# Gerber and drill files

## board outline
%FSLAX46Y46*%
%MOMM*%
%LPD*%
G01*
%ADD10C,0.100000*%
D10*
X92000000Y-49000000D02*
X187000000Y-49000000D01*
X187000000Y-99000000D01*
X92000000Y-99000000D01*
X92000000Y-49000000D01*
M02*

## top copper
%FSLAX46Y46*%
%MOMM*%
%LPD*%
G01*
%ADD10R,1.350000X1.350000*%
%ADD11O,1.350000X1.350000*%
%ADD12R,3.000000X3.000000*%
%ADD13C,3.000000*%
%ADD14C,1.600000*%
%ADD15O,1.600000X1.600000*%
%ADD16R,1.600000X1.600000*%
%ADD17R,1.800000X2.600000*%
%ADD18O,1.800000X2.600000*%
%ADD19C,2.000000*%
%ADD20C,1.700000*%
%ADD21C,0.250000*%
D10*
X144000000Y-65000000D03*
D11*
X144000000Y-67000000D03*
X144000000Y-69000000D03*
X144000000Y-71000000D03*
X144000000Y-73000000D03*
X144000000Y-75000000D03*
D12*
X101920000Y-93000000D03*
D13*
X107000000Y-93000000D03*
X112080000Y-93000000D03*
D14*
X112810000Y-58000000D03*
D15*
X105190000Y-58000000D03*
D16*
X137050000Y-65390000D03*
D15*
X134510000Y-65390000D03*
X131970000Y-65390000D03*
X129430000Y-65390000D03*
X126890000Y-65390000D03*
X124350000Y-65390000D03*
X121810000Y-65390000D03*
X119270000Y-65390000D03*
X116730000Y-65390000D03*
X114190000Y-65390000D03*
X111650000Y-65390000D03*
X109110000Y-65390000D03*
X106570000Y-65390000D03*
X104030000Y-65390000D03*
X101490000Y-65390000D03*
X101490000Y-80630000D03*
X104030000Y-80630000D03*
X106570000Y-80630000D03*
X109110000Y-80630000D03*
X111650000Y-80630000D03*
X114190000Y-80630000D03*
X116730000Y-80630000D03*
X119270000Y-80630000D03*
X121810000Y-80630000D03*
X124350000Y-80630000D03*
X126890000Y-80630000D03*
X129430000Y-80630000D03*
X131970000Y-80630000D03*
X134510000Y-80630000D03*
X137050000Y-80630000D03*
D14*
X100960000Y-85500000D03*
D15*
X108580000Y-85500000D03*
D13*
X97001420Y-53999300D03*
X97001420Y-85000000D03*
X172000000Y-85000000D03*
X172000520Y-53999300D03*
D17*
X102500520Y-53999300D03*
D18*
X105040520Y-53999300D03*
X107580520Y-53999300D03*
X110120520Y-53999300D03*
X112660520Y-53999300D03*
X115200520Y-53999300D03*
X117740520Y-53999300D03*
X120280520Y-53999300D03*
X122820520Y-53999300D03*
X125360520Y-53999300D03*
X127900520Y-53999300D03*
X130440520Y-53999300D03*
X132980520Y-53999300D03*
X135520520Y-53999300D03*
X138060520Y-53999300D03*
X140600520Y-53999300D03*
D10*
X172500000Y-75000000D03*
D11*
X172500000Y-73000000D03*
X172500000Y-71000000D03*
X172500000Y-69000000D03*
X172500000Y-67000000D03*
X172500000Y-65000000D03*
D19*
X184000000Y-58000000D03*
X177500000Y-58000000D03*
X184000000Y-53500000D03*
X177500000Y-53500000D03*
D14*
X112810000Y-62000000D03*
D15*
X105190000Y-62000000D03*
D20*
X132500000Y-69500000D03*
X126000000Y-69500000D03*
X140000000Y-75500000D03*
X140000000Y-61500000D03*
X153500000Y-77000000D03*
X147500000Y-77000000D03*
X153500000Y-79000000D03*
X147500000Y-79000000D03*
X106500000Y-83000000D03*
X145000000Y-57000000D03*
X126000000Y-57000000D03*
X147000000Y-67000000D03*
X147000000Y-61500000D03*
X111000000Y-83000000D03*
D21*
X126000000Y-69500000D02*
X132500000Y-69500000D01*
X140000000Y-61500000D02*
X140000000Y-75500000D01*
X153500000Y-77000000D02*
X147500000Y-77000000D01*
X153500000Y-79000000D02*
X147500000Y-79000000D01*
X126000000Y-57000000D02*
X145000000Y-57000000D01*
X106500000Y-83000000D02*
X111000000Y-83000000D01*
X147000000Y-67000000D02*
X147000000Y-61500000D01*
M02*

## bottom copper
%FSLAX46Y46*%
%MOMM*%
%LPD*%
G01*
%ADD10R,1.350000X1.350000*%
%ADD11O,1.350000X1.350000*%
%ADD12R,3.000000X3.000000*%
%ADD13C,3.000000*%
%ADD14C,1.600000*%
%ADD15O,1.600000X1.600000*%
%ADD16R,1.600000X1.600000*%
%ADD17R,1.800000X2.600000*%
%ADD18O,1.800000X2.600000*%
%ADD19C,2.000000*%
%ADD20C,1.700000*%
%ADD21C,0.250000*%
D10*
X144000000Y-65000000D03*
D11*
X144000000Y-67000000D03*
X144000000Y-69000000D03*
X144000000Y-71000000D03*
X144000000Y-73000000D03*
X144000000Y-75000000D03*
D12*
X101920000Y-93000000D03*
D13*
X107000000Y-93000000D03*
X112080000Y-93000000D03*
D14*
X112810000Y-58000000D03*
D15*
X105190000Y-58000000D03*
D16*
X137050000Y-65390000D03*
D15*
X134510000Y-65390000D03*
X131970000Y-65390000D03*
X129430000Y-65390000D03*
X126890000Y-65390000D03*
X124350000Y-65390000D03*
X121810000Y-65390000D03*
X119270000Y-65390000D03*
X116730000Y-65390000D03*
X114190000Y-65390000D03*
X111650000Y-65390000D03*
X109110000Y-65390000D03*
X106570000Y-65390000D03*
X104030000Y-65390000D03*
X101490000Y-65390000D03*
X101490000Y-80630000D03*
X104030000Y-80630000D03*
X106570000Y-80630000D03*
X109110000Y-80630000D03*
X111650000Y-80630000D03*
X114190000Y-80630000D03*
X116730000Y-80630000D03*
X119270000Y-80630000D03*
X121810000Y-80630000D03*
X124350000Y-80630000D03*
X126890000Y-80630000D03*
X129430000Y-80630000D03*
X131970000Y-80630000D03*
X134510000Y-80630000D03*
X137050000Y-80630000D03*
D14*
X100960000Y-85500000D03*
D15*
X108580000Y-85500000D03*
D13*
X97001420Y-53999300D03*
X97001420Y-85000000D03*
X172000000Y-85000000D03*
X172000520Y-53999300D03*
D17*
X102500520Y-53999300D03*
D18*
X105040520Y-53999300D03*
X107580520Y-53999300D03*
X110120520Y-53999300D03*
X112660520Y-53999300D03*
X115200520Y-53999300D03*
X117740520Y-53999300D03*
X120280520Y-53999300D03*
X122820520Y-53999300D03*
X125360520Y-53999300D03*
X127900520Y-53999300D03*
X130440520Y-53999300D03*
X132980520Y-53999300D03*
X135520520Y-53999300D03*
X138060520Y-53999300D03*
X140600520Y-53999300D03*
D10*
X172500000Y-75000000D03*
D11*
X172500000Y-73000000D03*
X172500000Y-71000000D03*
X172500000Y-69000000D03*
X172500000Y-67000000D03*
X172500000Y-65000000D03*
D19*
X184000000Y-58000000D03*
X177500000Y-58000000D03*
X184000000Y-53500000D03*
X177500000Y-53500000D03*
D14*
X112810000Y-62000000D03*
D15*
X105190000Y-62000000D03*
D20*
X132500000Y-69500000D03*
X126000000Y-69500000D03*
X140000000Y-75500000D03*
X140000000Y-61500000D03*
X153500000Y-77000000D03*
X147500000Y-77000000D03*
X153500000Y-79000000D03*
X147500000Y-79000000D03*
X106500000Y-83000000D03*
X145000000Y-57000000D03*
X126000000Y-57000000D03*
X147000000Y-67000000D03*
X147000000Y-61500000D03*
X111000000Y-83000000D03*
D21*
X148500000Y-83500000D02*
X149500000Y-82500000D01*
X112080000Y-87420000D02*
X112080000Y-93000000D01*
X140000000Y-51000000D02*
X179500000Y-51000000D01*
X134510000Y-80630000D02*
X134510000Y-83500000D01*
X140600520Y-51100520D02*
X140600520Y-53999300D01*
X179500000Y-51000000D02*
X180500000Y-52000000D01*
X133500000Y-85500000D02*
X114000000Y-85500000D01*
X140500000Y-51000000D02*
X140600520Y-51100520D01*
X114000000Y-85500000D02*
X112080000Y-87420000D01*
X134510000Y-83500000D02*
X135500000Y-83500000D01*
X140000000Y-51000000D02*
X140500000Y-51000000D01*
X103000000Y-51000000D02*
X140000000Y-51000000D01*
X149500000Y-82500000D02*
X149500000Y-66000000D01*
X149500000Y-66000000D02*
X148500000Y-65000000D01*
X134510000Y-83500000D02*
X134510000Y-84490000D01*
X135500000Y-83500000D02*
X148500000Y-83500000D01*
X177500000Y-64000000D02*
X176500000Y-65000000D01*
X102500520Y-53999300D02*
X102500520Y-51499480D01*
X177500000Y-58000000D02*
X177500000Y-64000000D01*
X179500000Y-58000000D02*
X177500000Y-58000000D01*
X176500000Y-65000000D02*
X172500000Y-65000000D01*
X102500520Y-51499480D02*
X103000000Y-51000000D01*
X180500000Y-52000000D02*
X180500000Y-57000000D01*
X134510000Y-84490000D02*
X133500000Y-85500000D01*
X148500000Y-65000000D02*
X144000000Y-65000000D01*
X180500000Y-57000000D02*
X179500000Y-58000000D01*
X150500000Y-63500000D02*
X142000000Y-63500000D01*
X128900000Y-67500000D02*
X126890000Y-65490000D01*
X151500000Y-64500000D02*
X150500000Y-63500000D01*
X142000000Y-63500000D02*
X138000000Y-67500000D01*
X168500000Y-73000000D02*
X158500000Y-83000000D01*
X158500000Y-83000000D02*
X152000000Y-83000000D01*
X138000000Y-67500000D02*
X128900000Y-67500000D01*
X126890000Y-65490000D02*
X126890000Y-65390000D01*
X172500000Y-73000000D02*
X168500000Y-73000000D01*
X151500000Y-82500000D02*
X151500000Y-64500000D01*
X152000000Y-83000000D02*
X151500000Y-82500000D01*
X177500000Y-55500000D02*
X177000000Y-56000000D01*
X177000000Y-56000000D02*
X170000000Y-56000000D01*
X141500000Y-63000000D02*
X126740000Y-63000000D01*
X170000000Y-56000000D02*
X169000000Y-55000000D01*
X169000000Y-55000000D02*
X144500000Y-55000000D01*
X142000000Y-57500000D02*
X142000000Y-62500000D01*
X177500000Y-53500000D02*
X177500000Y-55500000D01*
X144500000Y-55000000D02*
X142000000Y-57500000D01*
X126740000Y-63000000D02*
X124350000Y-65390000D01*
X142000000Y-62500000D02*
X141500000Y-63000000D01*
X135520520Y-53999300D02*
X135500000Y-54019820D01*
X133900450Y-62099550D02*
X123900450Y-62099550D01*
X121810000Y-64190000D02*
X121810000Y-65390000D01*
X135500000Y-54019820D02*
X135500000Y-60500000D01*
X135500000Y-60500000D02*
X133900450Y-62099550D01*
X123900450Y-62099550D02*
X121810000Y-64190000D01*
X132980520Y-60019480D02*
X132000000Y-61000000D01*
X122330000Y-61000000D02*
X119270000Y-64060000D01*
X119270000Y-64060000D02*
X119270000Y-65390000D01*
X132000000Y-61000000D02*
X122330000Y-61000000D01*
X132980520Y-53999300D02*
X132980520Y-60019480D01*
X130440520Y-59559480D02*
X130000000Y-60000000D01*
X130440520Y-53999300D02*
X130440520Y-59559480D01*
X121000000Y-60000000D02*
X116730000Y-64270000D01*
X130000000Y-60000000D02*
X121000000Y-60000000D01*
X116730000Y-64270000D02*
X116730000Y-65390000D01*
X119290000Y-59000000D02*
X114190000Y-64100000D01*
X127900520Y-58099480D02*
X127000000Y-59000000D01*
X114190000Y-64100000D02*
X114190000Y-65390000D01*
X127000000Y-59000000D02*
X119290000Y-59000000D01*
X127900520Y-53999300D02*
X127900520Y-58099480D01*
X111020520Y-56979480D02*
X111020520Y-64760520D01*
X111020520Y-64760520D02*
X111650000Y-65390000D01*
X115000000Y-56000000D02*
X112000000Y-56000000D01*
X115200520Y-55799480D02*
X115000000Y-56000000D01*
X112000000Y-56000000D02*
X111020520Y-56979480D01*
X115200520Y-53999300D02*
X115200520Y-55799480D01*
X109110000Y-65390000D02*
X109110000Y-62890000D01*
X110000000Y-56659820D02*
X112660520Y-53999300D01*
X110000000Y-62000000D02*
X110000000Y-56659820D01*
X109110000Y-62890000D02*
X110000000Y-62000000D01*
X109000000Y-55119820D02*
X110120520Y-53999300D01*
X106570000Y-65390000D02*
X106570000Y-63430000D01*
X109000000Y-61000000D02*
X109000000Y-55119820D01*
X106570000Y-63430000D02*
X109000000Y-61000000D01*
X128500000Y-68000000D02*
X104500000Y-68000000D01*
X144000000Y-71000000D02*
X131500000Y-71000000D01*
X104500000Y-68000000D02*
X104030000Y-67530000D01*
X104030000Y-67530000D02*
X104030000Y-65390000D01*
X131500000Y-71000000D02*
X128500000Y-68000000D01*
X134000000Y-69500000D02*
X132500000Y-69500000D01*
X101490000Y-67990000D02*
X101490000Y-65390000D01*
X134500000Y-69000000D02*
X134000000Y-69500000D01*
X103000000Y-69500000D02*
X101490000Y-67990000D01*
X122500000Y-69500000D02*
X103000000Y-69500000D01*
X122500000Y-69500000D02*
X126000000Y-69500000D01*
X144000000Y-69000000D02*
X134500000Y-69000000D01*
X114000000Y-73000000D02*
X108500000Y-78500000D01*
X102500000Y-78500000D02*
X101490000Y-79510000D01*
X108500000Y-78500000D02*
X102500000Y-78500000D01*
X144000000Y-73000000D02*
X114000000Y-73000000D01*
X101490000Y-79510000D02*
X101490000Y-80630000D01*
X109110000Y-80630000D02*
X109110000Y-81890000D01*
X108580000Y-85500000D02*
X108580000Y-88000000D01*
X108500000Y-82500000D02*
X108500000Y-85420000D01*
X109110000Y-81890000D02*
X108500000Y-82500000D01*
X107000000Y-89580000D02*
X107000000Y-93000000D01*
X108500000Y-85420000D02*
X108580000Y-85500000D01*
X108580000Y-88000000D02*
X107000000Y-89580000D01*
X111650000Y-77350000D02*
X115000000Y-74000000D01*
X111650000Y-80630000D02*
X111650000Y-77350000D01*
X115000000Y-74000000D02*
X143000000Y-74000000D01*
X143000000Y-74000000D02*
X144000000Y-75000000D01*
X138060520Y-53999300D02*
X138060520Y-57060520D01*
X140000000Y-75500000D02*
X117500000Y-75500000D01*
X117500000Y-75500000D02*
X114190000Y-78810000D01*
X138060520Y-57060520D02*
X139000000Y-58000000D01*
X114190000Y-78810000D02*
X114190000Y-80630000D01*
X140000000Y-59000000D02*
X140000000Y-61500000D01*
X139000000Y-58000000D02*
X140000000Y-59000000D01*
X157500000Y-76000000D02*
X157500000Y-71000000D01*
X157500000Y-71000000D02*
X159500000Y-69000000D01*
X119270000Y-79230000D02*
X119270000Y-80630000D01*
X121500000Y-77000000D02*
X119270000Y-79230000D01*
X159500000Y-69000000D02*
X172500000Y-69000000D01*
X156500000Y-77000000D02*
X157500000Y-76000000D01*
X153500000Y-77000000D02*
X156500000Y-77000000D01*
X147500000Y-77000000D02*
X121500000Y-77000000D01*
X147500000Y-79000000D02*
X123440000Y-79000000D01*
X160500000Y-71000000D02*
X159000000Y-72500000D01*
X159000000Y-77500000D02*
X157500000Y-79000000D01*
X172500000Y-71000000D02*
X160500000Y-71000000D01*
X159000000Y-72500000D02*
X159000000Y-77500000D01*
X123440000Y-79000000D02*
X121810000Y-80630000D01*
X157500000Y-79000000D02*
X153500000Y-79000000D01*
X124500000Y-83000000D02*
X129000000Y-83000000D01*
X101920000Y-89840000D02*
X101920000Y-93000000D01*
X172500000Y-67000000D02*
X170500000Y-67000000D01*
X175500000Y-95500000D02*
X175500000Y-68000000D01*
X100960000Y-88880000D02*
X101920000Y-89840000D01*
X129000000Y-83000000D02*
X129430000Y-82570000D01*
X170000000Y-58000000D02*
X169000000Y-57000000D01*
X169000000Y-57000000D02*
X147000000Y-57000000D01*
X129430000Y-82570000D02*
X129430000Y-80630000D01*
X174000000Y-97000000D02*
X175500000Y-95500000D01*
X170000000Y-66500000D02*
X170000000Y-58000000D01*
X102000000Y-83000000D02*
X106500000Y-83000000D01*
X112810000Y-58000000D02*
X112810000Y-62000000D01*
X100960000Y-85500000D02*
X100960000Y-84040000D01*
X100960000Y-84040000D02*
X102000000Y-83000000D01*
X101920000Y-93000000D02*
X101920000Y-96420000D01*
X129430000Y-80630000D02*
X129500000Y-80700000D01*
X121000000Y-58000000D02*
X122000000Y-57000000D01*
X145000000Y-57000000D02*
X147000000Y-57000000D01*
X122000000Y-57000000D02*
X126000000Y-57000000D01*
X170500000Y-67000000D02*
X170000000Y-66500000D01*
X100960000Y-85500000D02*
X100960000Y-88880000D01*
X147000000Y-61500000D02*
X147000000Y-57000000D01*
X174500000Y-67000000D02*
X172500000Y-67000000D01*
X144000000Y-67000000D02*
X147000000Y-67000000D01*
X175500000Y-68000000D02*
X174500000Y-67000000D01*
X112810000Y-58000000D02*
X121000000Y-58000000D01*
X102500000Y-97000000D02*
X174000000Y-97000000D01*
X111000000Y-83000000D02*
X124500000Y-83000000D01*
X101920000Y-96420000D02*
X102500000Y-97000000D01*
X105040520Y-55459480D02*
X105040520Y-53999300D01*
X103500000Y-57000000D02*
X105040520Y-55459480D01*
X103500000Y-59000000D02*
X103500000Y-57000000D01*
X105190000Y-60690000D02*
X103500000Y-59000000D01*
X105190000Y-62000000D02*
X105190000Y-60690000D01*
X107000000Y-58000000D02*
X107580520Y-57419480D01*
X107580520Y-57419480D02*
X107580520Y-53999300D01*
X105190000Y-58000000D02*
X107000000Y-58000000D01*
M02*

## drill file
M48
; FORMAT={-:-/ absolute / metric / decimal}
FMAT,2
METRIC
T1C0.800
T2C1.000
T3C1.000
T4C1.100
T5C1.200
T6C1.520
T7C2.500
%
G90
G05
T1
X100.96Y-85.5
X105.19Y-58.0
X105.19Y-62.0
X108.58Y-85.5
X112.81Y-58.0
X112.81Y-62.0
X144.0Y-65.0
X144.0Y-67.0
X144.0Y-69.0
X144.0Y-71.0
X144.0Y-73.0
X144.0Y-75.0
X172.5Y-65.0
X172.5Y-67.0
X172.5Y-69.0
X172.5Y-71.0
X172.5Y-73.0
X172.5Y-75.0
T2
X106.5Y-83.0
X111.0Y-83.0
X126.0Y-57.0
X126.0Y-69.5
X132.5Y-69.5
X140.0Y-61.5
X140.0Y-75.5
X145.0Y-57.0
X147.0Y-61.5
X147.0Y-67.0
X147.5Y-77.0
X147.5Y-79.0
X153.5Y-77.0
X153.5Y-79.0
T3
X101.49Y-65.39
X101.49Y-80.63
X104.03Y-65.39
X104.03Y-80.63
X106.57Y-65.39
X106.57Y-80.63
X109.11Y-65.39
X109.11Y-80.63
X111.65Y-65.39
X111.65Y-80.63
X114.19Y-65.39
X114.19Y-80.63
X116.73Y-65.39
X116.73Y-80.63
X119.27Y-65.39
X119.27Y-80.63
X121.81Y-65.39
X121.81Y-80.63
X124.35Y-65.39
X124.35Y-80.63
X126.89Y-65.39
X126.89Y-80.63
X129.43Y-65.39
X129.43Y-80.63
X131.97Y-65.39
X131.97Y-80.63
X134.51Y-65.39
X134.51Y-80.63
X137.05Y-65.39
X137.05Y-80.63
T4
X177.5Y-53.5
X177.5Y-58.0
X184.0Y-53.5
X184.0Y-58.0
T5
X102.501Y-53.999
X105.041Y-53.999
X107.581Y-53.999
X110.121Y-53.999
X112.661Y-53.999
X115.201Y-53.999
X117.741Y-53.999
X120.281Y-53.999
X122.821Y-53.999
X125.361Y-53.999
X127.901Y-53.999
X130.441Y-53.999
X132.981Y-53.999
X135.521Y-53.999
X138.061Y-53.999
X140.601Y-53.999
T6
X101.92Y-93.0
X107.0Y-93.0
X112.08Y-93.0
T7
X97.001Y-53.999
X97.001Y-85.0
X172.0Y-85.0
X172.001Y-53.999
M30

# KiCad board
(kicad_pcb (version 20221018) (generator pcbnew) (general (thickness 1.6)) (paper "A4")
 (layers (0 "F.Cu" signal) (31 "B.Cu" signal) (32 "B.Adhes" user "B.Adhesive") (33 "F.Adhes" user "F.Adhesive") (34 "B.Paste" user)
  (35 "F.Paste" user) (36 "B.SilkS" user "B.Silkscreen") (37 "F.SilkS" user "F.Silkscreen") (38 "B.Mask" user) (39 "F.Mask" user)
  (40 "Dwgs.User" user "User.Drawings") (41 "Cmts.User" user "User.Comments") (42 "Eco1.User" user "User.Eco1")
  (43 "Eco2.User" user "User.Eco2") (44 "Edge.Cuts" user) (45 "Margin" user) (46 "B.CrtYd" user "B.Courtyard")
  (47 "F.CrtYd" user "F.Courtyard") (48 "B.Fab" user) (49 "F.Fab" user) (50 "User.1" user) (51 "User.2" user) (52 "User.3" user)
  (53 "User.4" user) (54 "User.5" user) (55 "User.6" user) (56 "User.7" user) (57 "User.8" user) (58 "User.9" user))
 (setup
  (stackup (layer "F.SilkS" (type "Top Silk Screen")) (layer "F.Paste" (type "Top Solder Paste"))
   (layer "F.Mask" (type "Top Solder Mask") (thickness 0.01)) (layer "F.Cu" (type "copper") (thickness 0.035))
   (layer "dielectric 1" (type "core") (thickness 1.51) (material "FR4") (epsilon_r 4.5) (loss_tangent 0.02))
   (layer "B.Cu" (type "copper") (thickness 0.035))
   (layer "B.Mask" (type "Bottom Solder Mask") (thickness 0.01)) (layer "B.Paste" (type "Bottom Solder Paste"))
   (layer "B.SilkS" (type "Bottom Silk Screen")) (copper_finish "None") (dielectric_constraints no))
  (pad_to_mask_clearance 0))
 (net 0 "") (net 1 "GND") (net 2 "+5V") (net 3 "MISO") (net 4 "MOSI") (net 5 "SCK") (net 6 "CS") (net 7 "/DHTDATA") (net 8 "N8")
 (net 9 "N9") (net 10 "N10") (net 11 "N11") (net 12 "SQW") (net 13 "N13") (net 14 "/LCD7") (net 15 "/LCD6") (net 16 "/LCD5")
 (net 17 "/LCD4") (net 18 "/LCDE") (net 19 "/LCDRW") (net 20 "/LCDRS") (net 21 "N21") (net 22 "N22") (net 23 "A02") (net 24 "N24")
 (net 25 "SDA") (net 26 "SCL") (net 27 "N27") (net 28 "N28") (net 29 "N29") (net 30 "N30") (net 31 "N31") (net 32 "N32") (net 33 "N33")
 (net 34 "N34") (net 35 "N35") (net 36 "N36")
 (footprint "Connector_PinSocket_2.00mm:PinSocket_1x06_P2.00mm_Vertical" (layer "F.Cu") (at 144 65)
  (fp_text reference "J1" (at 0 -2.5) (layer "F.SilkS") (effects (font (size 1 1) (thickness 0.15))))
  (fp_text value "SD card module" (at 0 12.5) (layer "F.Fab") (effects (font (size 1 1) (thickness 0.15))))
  (pad "1" thru_hole rect (at 0 0) (size 1.35 1.35) (drill 0.8) (layers "*.Cu" "*.Mask") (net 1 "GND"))
  (pad "2" thru_hole oval (at 0 2) (size 1.35 1.35) (drill 0.8) (layers "*.Cu" "*.Mask") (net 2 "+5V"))
  (pad "3" thru_hole oval (at 0 4) (size 1.35 1.35) (drill 0.8) (layers "*.Cu" "*.Mask") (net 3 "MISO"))
  (pad "4" thru_hole oval (at 0 6) (size 1.35 1.35) (drill 0.8) (layers "*.Cu" "*.Mask") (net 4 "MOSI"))
  (pad "5" thru_hole oval (at 0 8) (size 1.35 1.35) (drill 0.8) (layers "*.Cu" "*.Mask") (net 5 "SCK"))
  (pad "6" thru_hole oval (at 0 10) (size 1.35 1.35) (drill 0.8) (layers "*.Cu" "*.Mask") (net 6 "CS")))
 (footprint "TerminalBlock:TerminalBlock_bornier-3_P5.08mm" (layer "F.Cu") (at 101.92 93)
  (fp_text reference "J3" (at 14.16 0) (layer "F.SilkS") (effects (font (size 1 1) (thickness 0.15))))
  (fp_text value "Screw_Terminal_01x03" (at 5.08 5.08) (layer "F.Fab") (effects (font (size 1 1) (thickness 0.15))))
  (pad "1" thru_hole rect (at 0 0) (size 3 3) (drill 1.52) (layers "*.Cu" "*.Mask") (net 2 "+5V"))
  (pad "2" thru_hole circle (at 5.08 0) (size 3 3) (drill 1.52) (layers "*.Cu" "*.Mask") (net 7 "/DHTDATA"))
  (pad "3" thru_hole circle (at 10.16 0) (size 3 3) (drill 1.52) (layers "*.Cu" "*.Mask") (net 1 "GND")))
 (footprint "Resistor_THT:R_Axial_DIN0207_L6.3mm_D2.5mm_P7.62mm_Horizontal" (layer "F.Cu") (at 112.81 58 180)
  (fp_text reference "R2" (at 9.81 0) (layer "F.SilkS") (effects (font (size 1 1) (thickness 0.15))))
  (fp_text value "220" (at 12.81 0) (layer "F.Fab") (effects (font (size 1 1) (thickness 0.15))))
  (pad "1" thru_hole circle (at 0 0 180) (size 1.6 1.6) (drill 0.8) (layers "*.Cu" "*.Mask") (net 2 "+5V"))
  (pad "2" thru_hole oval (at 7.62 0 180) (size 1.6 1.6) (drill 0.8) (layers "*.Cu" "*.Mask") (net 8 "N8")))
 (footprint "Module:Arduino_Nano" (layer "F.Cu") (at 137.05 65.39 -90)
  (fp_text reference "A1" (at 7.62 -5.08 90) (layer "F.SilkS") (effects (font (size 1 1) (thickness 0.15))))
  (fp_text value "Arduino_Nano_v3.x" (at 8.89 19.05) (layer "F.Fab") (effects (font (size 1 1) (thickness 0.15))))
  (pad "1" thru_hole rect (at 0 0 270) (size 1.6 1.6) (drill 1) (layers "*.Cu" "*.Mask") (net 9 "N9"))
  (pad "2" thru_hole oval (at 0 2.54 270) (size 1.6 1.6) (drill 1) (layers "*.Cu" "*.Mask") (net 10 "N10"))
  (pad "3" thru_hole oval (at 0 5.08 270) (size 1.6 1.6) (drill 1) (layers "*.Cu" "*.Mask") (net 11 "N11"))
  (pad "4" thru_hole oval (at 0 7.62 270) (size 1.6 1.6) (drill 1) (layers "*.Cu" "*.Mask") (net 1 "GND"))
  (pad "5" thru_hole oval (at 0 10.16 270) (size 1.6 1.6) (drill 1) (layers "*.Cu" "*.Mask") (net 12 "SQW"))
  (pad "6" thru_hole oval (at 0 12.7 270) (size 1.6 1.6) (drill 1) (layers "*.Cu" "*.Mask") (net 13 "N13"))
  (pad "7" thru_hole oval (at 0 15.24 270) (size 1.6 1.6) (drill 1) (layers "*.Cu" "*.Mask") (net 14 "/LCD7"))
  (pad "8" thru_hole oval (at 0 17.78 270) (size 1.6 1.6) (drill 1) (layers "*.Cu" "*.Mask") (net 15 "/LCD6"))
  (pad "9" thru_hole oval (at 0 20.32 270) (size 1.6 1.6) (drill 1) (layers "*.Cu" "*.Mask") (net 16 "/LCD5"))
  (pad "10" thru_hole oval (at 0 22.86 270) (size 1.6 1.6) (drill 1) (layers "*.Cu" "*.Mask") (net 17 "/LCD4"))
  (pad "11" thru_hole oval (at 0 25.4 270) (size 1.6 1.6) (drill 1) (layers "*.Cu" "*.Mask") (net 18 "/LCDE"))
  (pad "12" thru_hole oval (at 0 27.94 270) (size 1.6 1.6) (drill 1) (layers "*.Cu" "*.Mask") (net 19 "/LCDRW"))
  (pad "13" thru_hole oval (at 0 30.48 270) (size 1.6 1.6) (drill 1) (layers "*.Cu" "*.Mask") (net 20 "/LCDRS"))
  (pad "14" thru_hole oval (at 0 33.02 270) (size 1.6 1.6) (drill 1) (layers "*.Cu" "*.Mask") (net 4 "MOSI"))
  (pad "15" thru_hole oval (at 0 35.56 270) (size 1.6 1.6) (drill 1) (layers "*.Cu" "*.Mask") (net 3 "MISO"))
  (pad "16" thru_hole oval (at 15.24 35.56 270) (size 1.6 1.6) (drill 1) (layers "*.Cu" "*.Mask") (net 5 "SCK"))
  (pad "17" thru_hole oval (at 15.24 33.02 270) (size 1.6 1.6) (drill 1) (layers "*.Cu" "*.Mask") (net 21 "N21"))
  (pad "18" thru_hole oval (at 15.24 30.48 270) (size 1.6 1.6) (drill 1) (layers "*.Cu" "*.Mask") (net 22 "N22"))
  (pad "19" thru_hole oval (at 15.24 27.94 270) (size 1.6 1.6) (drill 1) (layers "*.Cu" "*.Mask") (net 7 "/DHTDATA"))
  (pad "20" thru_hole oval (at 15.24 25.4 270) (size 1.6 1.6) (drill 1) (layers "*.Cu" "*.Mask") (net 6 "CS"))
  (pad "21" thru_hole oval (at 15.24 22.86 270) (size 1.6 1.6) (drill 1) (layers "*.Cu" "*.Mask") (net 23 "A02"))
  (pad "22" thru_hole oval (at 15.24 20.32 270) (size 1.6 1.6) (drill 1) (layers "*.Cu" "*.Mask") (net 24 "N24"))
  (pad "23" thru_hole oval (at 15.24 17.78 270) (size 1.6 1.6) (drill 1) (layers "*.Cu" "*.Mask") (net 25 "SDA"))
  (pad "24" thru_hole oval (at 15.24 15.24 270) (size 1.6 1.6) (drill 1) (layers "*.Cu" "*.Mask") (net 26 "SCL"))
  (pad "25" thru_hole oval (at 15.24 12.7 270) (size 1.6 1.6) (drill 1) (layers "*.Cu" "*.Mask") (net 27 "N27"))
  (pad "26" thru_hole oval (at 15.24 10.16 270) (size 1.6 1.6) (drill 1) (layers "*.Cu" "*.Mask") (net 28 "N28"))
  (pad "27" thru_hole oval (at 15.24 7.62 270) (size 1.6 1.6) (drill 1) (layers "*.Cu" "*.Mask") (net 2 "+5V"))
  (pad "28" thru_hole oval (at 15.24 5.08 270) (size 1.6 1.6) (drill 1) (layers "*.Cu" "*.Mask") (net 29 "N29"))
  (pad "29" thru_hole oval (at 15.24 2.54 270) (size 1.6 1.6) (drill 1) (layers "*.Cu" "*.Mask") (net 1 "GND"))
  (pad "30" thru_hole oval (at 15.24 0 270) (size 1.6 1.6) (drill 1) (layers "*.Cu" "*.Mask") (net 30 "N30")))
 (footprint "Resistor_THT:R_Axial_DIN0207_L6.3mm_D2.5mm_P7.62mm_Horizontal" (layer "F.Cu") (at 100.96 85.5)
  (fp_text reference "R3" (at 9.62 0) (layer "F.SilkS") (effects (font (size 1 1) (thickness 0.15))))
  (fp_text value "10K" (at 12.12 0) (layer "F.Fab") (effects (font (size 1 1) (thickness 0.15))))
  (pad "1" thru_hole circle (at 0 0) (size 1.6 1.6) (drill 0.8) (layers "*.Cu" "*.Mask") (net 2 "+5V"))
  (pad "2" thru_hole oval (at 7.62 0) (size 1.6 1.6) (drill 0.8) (layers "*.Cu" "*.Mask") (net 7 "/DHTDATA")))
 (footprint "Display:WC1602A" (layer "F.Cu") (at 102.50052 53.9993)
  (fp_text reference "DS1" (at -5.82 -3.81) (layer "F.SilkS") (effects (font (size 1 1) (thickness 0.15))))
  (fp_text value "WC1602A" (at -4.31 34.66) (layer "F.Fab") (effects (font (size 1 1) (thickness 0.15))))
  (pad "" thru_hole circle (at -5.4991 0) (size 3 3) (drill 2.5) (layers "*.Cu" "*.Mask"))
  (pad "" thru_hole circle (at -5.4991 31.0007) (size 3 3) (drill 2.5) (layers "*.Cu" "*.Mask"))
  (pad "" thru_hole circle (at 69.49948 31.0007) (size 3 3) (drill 2.5) (layers "*.Cu" "*.Mask"))
  (pad "" thru_hole circle (at 69.5 0) (size 3 3) (drill 2.5) (layers "*.Cu" "*.Mask"))
  (pad "1" thru_hole rect (at 0 0) (size 1.8 2.6) (drill 1.2) (layers "*.Cu" "*.Mask") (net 1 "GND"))
  (pad "2" thru_hole oval (at 2.54 0) (size 1.8 2.6) (drill 1.2) (layers "*.Cu" "*.Mask") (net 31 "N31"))
  (pad "3" thru_hole oval (at 5.08 0) (size 1.8 2.6) (drill 1.2) (layers "*.Cu" "*.Mask") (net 8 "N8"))
  (pad "4" thru_hole oval (at 7.62 0) (size 1.8 2.6) (drill 1.2) (layers "*.Cu" "*.Mask") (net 20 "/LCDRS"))
  (pad "5" thru_hole oval (at 10.16 0) (size 1.8 2.6) (drill 1.2) (layers "*.Cu" "*.Mask") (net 19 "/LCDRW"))
  (pad "6" thru_hole oval (at 12.7 0) (size 1.8 2.6) (drill 1.2) (layers "*.Cu" "*.Mask") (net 18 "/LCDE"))
  (pad "7" thru_hole oval (at 15.24 0) (size 1.8 2.6) (drill 1.2) (layers "*.Cu" "*.Mask") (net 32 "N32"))
  (pad "8" thru_hole oval (at 17.78 0) (size 1.8 2.6) (drill 1.2) (layers "*.Cu" "*.Mask") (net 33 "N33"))
  (pad "9" thru_hole oval (at 20.32 0) (size 1.8 2.6) (drill 1.2) (layers "*.Cu" "*.Mask") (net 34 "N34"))
  (pad "10" thru_hole oval (at 22.86 0) (size 1.8 2.6) (drill 1.2) (layers "*.Cu" "*.Mask") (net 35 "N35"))
  (pad "11" thru_hole oval (at 25.4 0) (size 1.8 2.6) (drill 1.2) (layers "*.Cu" "*.Mask") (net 17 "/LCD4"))
  (pad "12" thru_hole oval (at 27.94 0) (size 1.8 2.6) (drill 1.2) (layers "*.Cu" "*.Mask") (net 16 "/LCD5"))
  (pad "13" thru_hole oval (at 30.48 0) (size 1.8 2.6) (drill 1.2) (layers "*.Cu" "*.Mask") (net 15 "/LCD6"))
  (pad "14" thru_hole oval (at 33.02 0) (size 1.8 2.6) (drill 1.2) (layers "*.Cu" "*.Mask") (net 14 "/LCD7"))
  (pad "15" thru_hole oval (at 35.56 0) (size 1.8 2.6) (drill 1.2) (layers "*.Cu" "*.Mask") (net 23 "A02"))
  (pad "16" thru_hole oval (at 38.1 0) (size 1.8 2.6) (drill 1.2) (layers "*.Cu" "*.Mask") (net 1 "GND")))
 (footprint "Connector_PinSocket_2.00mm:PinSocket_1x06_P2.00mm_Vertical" (layer "F.Cu") (at 172.5 75 180)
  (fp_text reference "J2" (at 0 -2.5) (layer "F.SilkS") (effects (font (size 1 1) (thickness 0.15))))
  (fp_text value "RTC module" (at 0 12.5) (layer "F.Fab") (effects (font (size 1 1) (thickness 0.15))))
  (pad "1" thru_hole rect (at 0 0 180) (size 1.35 1.35) (drill 0.8) (layers "*.Cu" "*.Mask") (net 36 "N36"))
  (pad "2" thru_hole oval (at 0 2 180) (size 1.35 1.35) (drill 0.8) (layers "*.Cu" "*.Mask") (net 12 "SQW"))
  (pad "3" thru_hole oval (at 0 4 180) (size 1.35 1.35) (drill 0.8) (layers "*.Cu" "*.Mask") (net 26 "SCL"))
  (pad "4" thru_hole oval (at 0 6 180) (size 1.35 1.35) (drill 0.8) (layers "*.Cu" "*.Mask") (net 25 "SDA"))
  (pad "5" thru_hole oval (at 0 8 180) (size 1.35 1.35) (drill 0.8) (layers "*.Cu" "*.Mask") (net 2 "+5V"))
  (pad "6" thru_hole oval (at 0 10 180) (size 1.35 1.35) (drill 0.8) (layers "*.Cu" "*.Mask") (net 1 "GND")))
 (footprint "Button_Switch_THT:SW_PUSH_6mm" (layer "F.Cu") (at 184 58 180)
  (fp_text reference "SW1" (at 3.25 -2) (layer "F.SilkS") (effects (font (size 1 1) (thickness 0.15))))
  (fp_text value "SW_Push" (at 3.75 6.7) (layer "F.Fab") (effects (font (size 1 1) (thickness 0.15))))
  (pad "1" thru_hole circle (at 0 0 270) (size 2 2) (drill 1.1) (layers "*.Cu" "*.Mask") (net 1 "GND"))
  (pad "1" thru_hole circle (at 6.5 0 270) (size 2 2) (drill 1.1) (layers "*.Cu" "*.Mask") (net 1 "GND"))
  (pad "2" thru_hole circle (at 0 4.5 270) (size 2 2) (drill 1.1) (layers "*.Cu" "*.Mask") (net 13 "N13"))
  (pad "2" thru_hole circle (at 6.5 4.5 270) (size 2 2) (drill 1.1) (layers "*.Cu" "*.Mask") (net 13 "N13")))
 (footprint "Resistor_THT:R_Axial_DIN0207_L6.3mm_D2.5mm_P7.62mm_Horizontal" (layer "F.Cu") (at 112.81 62 180)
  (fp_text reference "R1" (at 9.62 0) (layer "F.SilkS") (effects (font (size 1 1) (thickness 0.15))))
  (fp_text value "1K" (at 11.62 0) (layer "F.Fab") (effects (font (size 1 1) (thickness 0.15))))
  (pad "1" thru_hole circle (at 0 0 180) (size 1.6 1.6) (drill 0.8) (layers "*.Cu" "*.Mask") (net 2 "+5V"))
  (pad "2" thru_hole oval (at 7.62 0 180) (size 1.6 1.6) (drill 0.8) (layers "*.Cu" "*.Mask") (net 31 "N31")))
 (gr_rect (start 92 49) (end 187 99) (stroke (width 0.1) (type default)) (fill none) (layer "Edge.Cuts"))
 (segment (start 148.5 83.5) (end 149.5 82.5) (width 0.25) (layer "B.Cu") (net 1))
 (segment (start 112.08 87.42) (end 112.08 93) (width 0.25) (layer "B.Cu") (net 1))
 (segment (start 140 51) (end 179.5 51) (width 0.25) (layer "B.Cu") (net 1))
 (segment (start 134.51 80.63) (end 134.51 83.5) (width 0.25) (layer "B.Cu") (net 1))
 (segment (start 140.60052 51.10052) (end 140.60052 53.9993) (width 0.25) (layer "B.Cu") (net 1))
 (segment (start 179.5 51) (end 180.5 52) (width 0.25) (layer "B.Cu") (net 1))
 (segment (start 133.5 85.5) (end 114 85.5) (width 0.25) (layer "B.Cu") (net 1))
 (segment (start 140.5 51) (end 140.60052 51.10052) (width 0.25) (layer "B.Cu") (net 1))
 (segment (start 114 85.5) (end 112.08 87.42) (width 0.25) (layer "B.Cu") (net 1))
 (segment (start 134.51 83.5) (end 135.5 83.5) (width 0.25) (layer "B.Cu") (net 1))
 (segment (start 140 51) (end 140.5 51) (width 0.25) (layer "B.Cu") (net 1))
 (segment (start 103 51) (end 140 51) (width 0.25) (layer "B.Cu") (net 1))
 (segment (start 149.5 82.5) (end 149.5 66) (width 0.25) (layer "B.Cu") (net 1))
 (segment (start 149.5 66) (end 148.5 65) (width 0.25) (layer "B.Cu") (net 1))
 (segment (start 134.51 83.5) (end 134.51 84.49) (width 0.25) (layer "B.Cu") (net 1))
 (segment (start 135.5 83.5) (end 148.5 83.5) (width 0.25) (layer "B.Cu") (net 1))
 (segment (start 177.5 64) (end 176.5 65) (width 0.25) (layer "B.Cu") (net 1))
 (segment (start 102.50052 53.9993) (end 102.50052 51.49948) (width 0.25) (layer "B.Cu") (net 1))
 (segment (start 177.5 58) (end 177.5 64) (width 0.25) (layer "B.Cu") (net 1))
 (segment (start 179.5 58) (end 177.5 58) (width 0.25) (layer "B.Cu") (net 1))
 (segment (start 176.5 65) (end 172.5 65) (width 0.25) (layer "B.Cu") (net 1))
 (segment (start 102.50052 51.49948) (end 103 51) (width 0.25) (layer "B.Cu") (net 1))
 (segment (start 180.5 52) (end 180.5 57) (width 0.25) (layer "B.Cu") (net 1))
 (segment (start 134.51 84.49) (end 133.5 85.5) (width 0.25) (layer "B.Cu") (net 1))
 (segment (start 148.5 65) (end 144 65) (width 0.25) (layer "B.Cu") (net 1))
 (segment (start 180.5 57) (end 179.5 58) (width 0.25) (layer "B.Cu") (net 1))
 (segment (start 150.5 63.5) (end 142 63.5) (width 0.25) (layer "B.Cu") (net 12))
 (segment (start 128.9 67.5) (end 126.89 65.49) (width 0.25) (layer "B.Cu") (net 12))
 (segment (start 151.5 64.5) (end 150.5 63.5) (width 0.25) (layer "B.Cu") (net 12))
 (segment (start 142 63.5) (end 138 67.5) (width 0.25) (layer "B.Cu") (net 12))
 (segment (start 168.5 73) (end 158.5 83) (width 0.25) (layer "B.Cu") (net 12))
 (segment (start 158.5 83) (end 152 83) (width 0.25) (layer "B.Cu") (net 12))
 (segment (start 138 67.5) (end 128.9 67.5) (width 0.25) (layer "B.Cu") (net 12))
 (segment (start 126.89 65.49) (end 126.89 65.39) (width 0.25) (layer "B.Cu") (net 12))
 (segment (start 172.5 73) (end 168.5 73) (width 0.25) (layer "B.Cu") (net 12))
 (segment (start 151.5 82.5) (end 151.5 64.5) (width 0.25) (layer "B.Cu") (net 12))
 (segment (start 152 83) (end 151.5 82.5) (width 0.25) (layer "B.Cu") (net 12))
 (segment (start 177.5 55.5) (end 177 56) (width 0.25) (layer "B.Cu") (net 13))
 (segment (start 177 56) (end 170 56) (width 0.25) (layer "B.Cu") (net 13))
 (segment (start 141.5 63) (end 126.74 63) (width 0.25) (layer "B.Cu") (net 13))
 (segment (start 170 56) (end 169 55) (width 0.25) (layer "B.Cu") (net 13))
 (segment (start 169 55) (end 144.5 55) (width 0.25) (layer "B.Cu") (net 13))
 (segment (start 142 57.5) (end 142 62.5) (width 0.25) (layer "B.Cu") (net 13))
 (segment (start 177.5 53.5) (end 177.5 55.5) (width 0.25) (layer "B.Cu") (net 13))
 (segment (start 144.5 55) (end 142 57.5) (width 0.25) (layer "B.Cu") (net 13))
 (segment (start 126.74 63) (end 124.35 65.39) (width 0.25) (layer "B.Cu") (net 13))
 (segment (start 142 62.5) (end 141.5 63) (width 0.25) (layer "B.Cu") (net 13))
 (segment (start 135.52052 53.9993) (end 135.5 54.01982) (width 0.25) (layer "B.Cu") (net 14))
 (segment (start 133.90045 62.09955) (end 123.90045 62.09955) (width 0.25) (layer "B.Cu") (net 14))
 (segment (start 121.81 64.19) (end 121.81 65.39) (width 0.25) (layer "B.Cu") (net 14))
 (segment (start 135.5 54.01982) (end 135.5 60.5) (width 0.25) (layer "B.Cu") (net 14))
 (segment (start 135.5 60.5) (end 133.90045 62.09955) (width 0.25) (layer "B.Cu") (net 14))
 (segment (start 123.90045 62.09955) (end 121.81 64.19) (width 0.25) (layer "B.Cu") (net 14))
 (segment (start 132.98052 60.01948) (end 132 61) (width 0.25) (layer "B.Cu") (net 15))
 (segment (start 122.33 61) (end 119.27 64.06) (width 0.25) (layer "B.Cu") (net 15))
 (segment (start 119.27 64.06) (end 119.27 65.39) (width 0.25) (layer "B.Cu") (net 15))
 (segment (start 132 61) (end 122.33 61) (width 0.25) (layer "B.Cu") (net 15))
 (segment (start 132.98052 53.9993) (end 132.98052 60.01948) (width 0.25) (layer "B.Cu") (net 15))
 (segment (start 130.44052 59.55948) (end 130 60) (width 0.25) (layer "B.Cu") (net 16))
 (segment (start 130.44052 53.9993) (end 130.44052 59.55948) (width 0.25) (layer "B.Cu") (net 16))
 (segment (start 121 60) (end 116.73 64.27) (width 0.25) (layer "B.Cu") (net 16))
 (segment (start 130 60) (end 121 60) (width 0.25) (layer "B.Cu") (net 16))
 (segment (start 116.73 64.27) (end 116.73 65.39) (width 0.25) (layer "B.Cu") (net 16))
 (segment (start 119.29 59) (end 114.19 64.1) (width 0.25) (layer "B.Cu") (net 17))
 (segment (start 127.90052 58.09948) (end 127 59) (width 0.25) (layer "B.Cu") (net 17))
 (segment (start 114.19 64.1) (end 114.19 65.39) (width 0.25) (layer "B.Cu") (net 17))
 (segment (start 127 59) (end 119.29 59) (width 0.25) (layer "B.Cu") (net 17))
 (segment (start 127.90052 53.9993) (end 127.90052 58.09948) (width 0.25) (layer "B.Cu") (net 17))
 (segment (start 111.02052 56.97948) (end 111.02052 64.76052) (width 0.25) (layer "B.Cu") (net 18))
 (segment (start 111.02052 64.76052) (end 111.65 65.39) (width 0.25) (layer "B.Cu") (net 18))
 (segment (start 115 56) (end 112 56) (width 0.25) (layer "B.Cu") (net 18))
 (segment (start 115.20052 55.79948) (end 115 56) (width 0.25) (layer "B.Cu") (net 18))
 (segment (start 112 56) (end 111.02052 56.97948) (width 0.25) (layer "B.Cu") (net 18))
 (segment (start 115.20052 53.9993) (end 115.20052 55.79948) (width 0.25) (layer "B.Cu") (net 18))
 (segment (start 109.11 65.39) (end 109.11 62.89) (width 0.25) (layer "B.Cu") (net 19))
 (segment (start 110 56.65982) (end 112.66052 53.9993) (width 0.25) (layer "B.Cu") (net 19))
 (segment (start 110 62) (end 110 56.65982) (width 0.25) (layer "B.Cu") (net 19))
 (segment (start 109.11 62.89) (end 110 62) (width 0.25) (layer "B.Cu") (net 19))
 (segment (start 109 55.11982) (end 110.12052 53.9993) (width 0.25) (layer "B.Cu") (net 20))
 (segment (start 106.57 65.39) (end 106.57 63.43) (width 0.25) (layer "B.Cu") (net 20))
 (segment (start 109 61) (end 109 55.11982) (width 0.25) (layer "B.Cu") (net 20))
 (segment (start 106.57 63.43) (end 109 61) (width 0.25) (layer "B.Cu") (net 20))
 (segment (start 128.5 68) (end 104.5 68) (width 0.25) (layer "B.Cu") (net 4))
 (segment (start 144 71) (end 131.5 71) (width 0.25) (layer "B.Cu") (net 4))
 (segment (start 104.5 68) (end 104.03 67.53) (width 0.25) (layer "B.Cu") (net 4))
 (segment (start 104.03 67.53) (end 104.03 65.39) (width 0.25) (layer "B.Cu") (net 4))
 (segment (start 131.5 71) (end 128.5 68) (width 0.25) (layer "B.Cu") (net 4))
 (segment (start 126 69.5) (end 132.5 69.5) (width 0.25) (layer "F.Cu") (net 3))
 (via (at 132.5 69.5) (size 1.7) (drill 1) (layers "F.Cu" "B.Cu") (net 3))
 (via (at 126 69.5) (size 1.7) (drill 1) (layers "F.Cu" "B.Cu") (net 3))
 (segment (start 134 69.5) (end 132.5 69.5) (width 0.25) (layer "B.Cu") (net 3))
 (segment (start 101.49 67.99) (end 101.49 65.39) (width 0.25) (layer "B.Cu") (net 3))
 (segment (start 134.5 69) (end 134 69.5) (width 0.25) (layer "B.Cu") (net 3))
 (segment (start 103 69.5) (end 101.49 67.99) (width 0.25) (layer "B.Cu") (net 3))
 (segment (start 122.5 69.5) (end 103 69.5) (width 0.25) (layer "B.Cu") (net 3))
 (segment (start 122.5 69.5) (end 126 69.5) (width 0.25) (layer "B.Cu") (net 3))
 (segment (start 144 69) (end 134.5 69) (width 0.25) (layer "B.Cu") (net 3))
 (segment (start 114 73) (end 108.5 78.5) (width 0.25) (layer "B.Cu") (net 5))
 (segment (start 102.5 78.5) (end 101.49 79.51) (width 0.25) (layer "B.Cu") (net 5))
 (segment (start 108.5 78.5) (end 102.5 78.5) (width 0.25) (layer "B.Cu") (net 5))
 (segment (start 144 73) (end 114 73) (width 0.25) (layer "B.Cu") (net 5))
 (segment (start 101.49 79.51) (end 101.49 80.63) (width 0.25) (layer "B.Cu") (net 5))
 (segment (start 109.11 80.63) (end 109.11 81.89) (width 0.25) (layer "B.Cu") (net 7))
 (segment (start 108.58 85.5) (end 108.58 88) (width 0.25) (layer "B.Cu") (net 7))
 (segment (start 108.5 82.5) (end 108.5 85.42) (width 0.25) (layer "B.Cu") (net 7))
 (segment (start 109.11 81.89) (end 108.5 82.5) (width 0.25) (layer "B.Cu") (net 7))
 (segment (start 107 89.58) (end 107 93) (width 0.25) (layer "B.Cu") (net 7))
 (segment (start 108.5 85.42) (end 108.58 85.5) (width 0.25) (layer "B.Cu") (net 7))
 (segment (start 108.58 88) (end 107 89.58) (width 0.25) (layer "B.Cu") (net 7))
 (segment (start 111.65 77.35) (end 115 74) (width 0.25) (layer "B.Cu") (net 6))
 (segment (start 111.65 80.63) (end 111.65 77.35) (width 0.25) (layer "B.Cu") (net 6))
 (segment (start 115 74) (end 143 74) (width 0.25) (layer "B.Cu") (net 6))
 (segment (start 143 74) (end 144 75) (width 0.25) (layer "B.Cu") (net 6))
 (segment (start 140 61.5) (end 140 75.5) (width 0.25) (layer "F.Cu") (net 23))
 (via (at 140 75.5) (size 1.7) (drill 1) (layers "F.Cu" "B.Cu") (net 23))
 (via (at 140 61.5) (size 1.7) (drill 1) (layers "F.Cu" "B.Cu") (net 23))
 (segment (start 138.06052 53.9993) (end 138.06052 57.06052) (width 0.25) (layer "B.Cu") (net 23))
 (segment (start 140 75.5) (end 117.5 75.5) (width 0.25) (layer "B.Cu") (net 23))
 (segment (start 117.5 75.5) (end 114.19 78.81) (width 0.25) (layer "B.Cu") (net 23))
 (segment (start 138.06052 57.06052) (end 139 58) (width 0.25) (layer "B.Cu") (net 23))
 (segment (start 114.19 78.81) (end 114.19 80.63) (width 0.25) (layer "B.Cu") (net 23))
 (segment (start 140 59) (end 140 61.5) (width 0.25) (layer "B.Cu") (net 23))
 (segment (start 139 58) (end 140 59) (width 0.25) (layer "B.Cu") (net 23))
 (segment (start 153.5 77) (end 147.5 77) (width 0.25) (layer "F.Cu") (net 25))
 (via (at 153.5 77) (size 1.7) (drill 1) (layers "F.Cu" "B.Cu") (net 25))
 (via (at 147.5 77) (size 1.7) (drill 1) (layers "F.Cu" "B.Cu") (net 25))
 (segment (start 157.5 76) (end 157.5 71) (width 0.25) (layer "B.Cu") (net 25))
 (segment (start 157.5 71) (end 159.5 69) (width 0.25) (layer "B.Cu") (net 25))
 (segment (start 119.27 79.23) (end 119.27 80.63) (width 0.25) (layer "B.Cu") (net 25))
 (segment (start 121.5 77) (end 119.27 79.23) (width 0.25) (layer "B.Cu") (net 25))
 (segment (start 159.5 69) (end 172.5 69) (width 0.25) (layer "B.Cu") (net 25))
 (segment (start 156.5 77) (end 157.5 76) (width 0.25) (layer "B.Cu") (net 25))
 (segment (start 153.5 77) (end 156.5 77) (width 0.25) (layer "B.Cu") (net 25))
 (segment (start 147.5 77) (end 121.5 77) (width 0.25) (layer "B.Cu") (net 25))
 (segment (start 153.5 79) (end 147.5 79) (width 0.25) (layer "F.Cu") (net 26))
 (via (at 153.5 79) (size 1.7) (drill 1) (layers "F.Cu" "B.Cu") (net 26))
 (via (at 147.5 79) (size 1.7) (drill 1) (layers "F.Cu" "B.Cu") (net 26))
 (segment (start 147.5 79) (end 123.44 79) (width 0.25) (layer "B.Cu") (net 26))
 (segment (start 160.5 71) (end 159 72.5) (width 0.25) (layer "B.Cu") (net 26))
 (segment (start 159 77.5) (end 157.5 79) (width 0.25) (layer "B.Cu") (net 26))
 (segment (start 172.5 71) (end 160.5 71) (width 0.25) (layer "B.Cu") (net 26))
 (segment (start 159 72.5) (end 159 77.5) (width 0.25) (layer "B.Cu") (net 26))
 (segment (start 123.44 79) (end 121.81 80.63) (width 0.25) (layer "B.Cu") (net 26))
 (segment (start 157.5 79) (end 153.5 79) (width 0.25) (layer "B.Cu") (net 26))
 (segment (start 126 57) (end 145 57) (width 0.25) (layer "F.Cu") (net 2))
 (segment (start 106.5 83) (end 111 83) (width 0.25) (layer "F.Cu") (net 2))
 (segment (start 147 67) (end 147 61.5) (width 0.25) (layer "F.Cu") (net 2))
 (via (at 106.5 83) (size 1.7) (drill 1) (layers "F.Cu" "B.Cu") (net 2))
 (via (at 145 57) (size 1.7) (drill 1) (layers "F.Cu" "B.Cu") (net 2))
 (via (at 126 57) (size 1.7) (drill 1) (layers "F.Cu" "B.Cu") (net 2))
 (via (at 147 67) (size 1.7) (drill 1) (layers "F.Cu" "B.Cu") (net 2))
 (via (at 147 61.5) (size 1.7) (drill 1) (layers "F.Cu" "B.Cu") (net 2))
 (via (at 111 83) (size 1.7) (drill 1) (layers "F.Cu" "B.Cu") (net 2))
 (segment (start 124.5 83) (end 129 83) (width 0.25) (layer "B.Cu") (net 2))
 (segment (start 101.92 89.84) (end 101.92 93) (width 0.25) (layer "B.Cu") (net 2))
 (segment (start 172.5 67) (end 170.5 67) (width 0.25) (layer "B.Cu") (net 2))
 (segment (start 175.5 95.5) (end 175.5 68) (width 0.25) (layer "B.Cu") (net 2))
 (segment (start 100.96 88.88) (end 101.92 89.84) (width 0.25) (layer "B.Cu") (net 2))
 (segment (start 129 83) (end 129.43 82.57) (width 0.25) (layer "B.Cu") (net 2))
 (segment (start 170 58) (end 169 57) (width 0.25) (layer "B.Cu") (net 2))
 (segment (start 169 57) (end 147 57) (width 0.25) (layer "B.Cu") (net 2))
 (segment (start 129.43 82.57) (end 129.43 80.63) (width 0.25) (layer "B.Cu") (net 2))
 (segment (start 174 97) (end 175.5 95.5) (width 0.25) (layer "B.Cu") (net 2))
 (segment (start 170 66.5) (end 170 58) (width 0.25) (layer "B.Cu") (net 2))
 (segment (start 102 83) (end 106.5 83) (width 0.25) (layer "B.Cu") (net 2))
 (segment (start 112.81 58) (end 112.81 62) (width 0.25) (layer "B.Cu") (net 2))
 (segment (start 100.96 85.5) (end 100.96 84.04) (width 0.25) (layer "B.Cu") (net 2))
 (segment (start 100.96 84.04) (end 102 83) (width 0.25) (layer "B.Cu") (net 2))
 (segment (start 101.92 93) (end 101.92 96.42) (width 0.25) (layer "B.Cu") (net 2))
 (segment (start 129.43 80.63) (end 129.5 80.7) (width 0.25) (layer "B.Cu") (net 2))
 (segment (start 121 58) (end 122 57) (width 0.25) (layer "B.Cu") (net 2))
 (segment (start 145 57) (end 147 57) (width 0.25) (layer "B.Cu") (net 2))
 (segment (start 122 57) (end 126 57) (width 0.25) (layer "B.Cu") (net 2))
 (segment (start 170.5 67) (end 170 66.5) (width 0.25) (layer "B.Cu") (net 2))
 (segment (start 100.96 85.5) (end 100.96 88.88) (width 0.25) (layer "B.Cu") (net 2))
 (segment (start 147 61.5) (end 147 57) (width 0.25) (layer "B.Cu") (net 2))
 (segment (start 174.5 67) (end 172.5 67) (width 0.25) (layer "B.Cu") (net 2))
 (segment (start 144 67) (end 147 67) (width 0.25) (layer "B.Cu") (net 2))
 (segment (start 175.5 68) (end 174.5 67) (width 0.25) (layer "B.Cu") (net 2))
 (segment (start 112.81 58) (end 121 58) (width 0.25) (layer "B.Cu") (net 2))
 (segment (start 102.5 97) (end 174 97) (width 0.25) (layer "B.Cu") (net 2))
 (segment (start 111 83) (end 124.5 83) (width 0.25) (layer "B.Cu") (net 2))
 (segment (start 101.92 96.42) (end 102.5 97) (width 0.25) (layer "B.Cu") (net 2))
 (segment (start 105.04052 55.45948) (end 105.04052 53.9993) (width 0.25) (layer "B.Cu") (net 31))
 (segment (start 103.5 57) (end 105.04052 55.45948) (width 0.25) (layer "B.Cu") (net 31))
 (segment (start 103.5 59) (end 103.5 57) (width 0.25) (layer "B.Cu") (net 31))
 (segment (start 105.19 60.69) (end 103.5 59) (width 0.25) (layer "B.Cu") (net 31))
 (segment (start 105.19 62) (end 105.19 60.69) (width 0.25) (layer "B.Cu") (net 31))
 (segment (start 107 58) (end 107.58052 57.41948) (width 0.25) (layer "B.Cu") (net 8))
 (segment (start 107.58052 57.41948) (end 107.58052 53.9993) (width 0.25) (layer "B.Cu") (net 8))
 (segment (start 105.19 58) (end 107 58) (width 0.25) (layer "B.Cu") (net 8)))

